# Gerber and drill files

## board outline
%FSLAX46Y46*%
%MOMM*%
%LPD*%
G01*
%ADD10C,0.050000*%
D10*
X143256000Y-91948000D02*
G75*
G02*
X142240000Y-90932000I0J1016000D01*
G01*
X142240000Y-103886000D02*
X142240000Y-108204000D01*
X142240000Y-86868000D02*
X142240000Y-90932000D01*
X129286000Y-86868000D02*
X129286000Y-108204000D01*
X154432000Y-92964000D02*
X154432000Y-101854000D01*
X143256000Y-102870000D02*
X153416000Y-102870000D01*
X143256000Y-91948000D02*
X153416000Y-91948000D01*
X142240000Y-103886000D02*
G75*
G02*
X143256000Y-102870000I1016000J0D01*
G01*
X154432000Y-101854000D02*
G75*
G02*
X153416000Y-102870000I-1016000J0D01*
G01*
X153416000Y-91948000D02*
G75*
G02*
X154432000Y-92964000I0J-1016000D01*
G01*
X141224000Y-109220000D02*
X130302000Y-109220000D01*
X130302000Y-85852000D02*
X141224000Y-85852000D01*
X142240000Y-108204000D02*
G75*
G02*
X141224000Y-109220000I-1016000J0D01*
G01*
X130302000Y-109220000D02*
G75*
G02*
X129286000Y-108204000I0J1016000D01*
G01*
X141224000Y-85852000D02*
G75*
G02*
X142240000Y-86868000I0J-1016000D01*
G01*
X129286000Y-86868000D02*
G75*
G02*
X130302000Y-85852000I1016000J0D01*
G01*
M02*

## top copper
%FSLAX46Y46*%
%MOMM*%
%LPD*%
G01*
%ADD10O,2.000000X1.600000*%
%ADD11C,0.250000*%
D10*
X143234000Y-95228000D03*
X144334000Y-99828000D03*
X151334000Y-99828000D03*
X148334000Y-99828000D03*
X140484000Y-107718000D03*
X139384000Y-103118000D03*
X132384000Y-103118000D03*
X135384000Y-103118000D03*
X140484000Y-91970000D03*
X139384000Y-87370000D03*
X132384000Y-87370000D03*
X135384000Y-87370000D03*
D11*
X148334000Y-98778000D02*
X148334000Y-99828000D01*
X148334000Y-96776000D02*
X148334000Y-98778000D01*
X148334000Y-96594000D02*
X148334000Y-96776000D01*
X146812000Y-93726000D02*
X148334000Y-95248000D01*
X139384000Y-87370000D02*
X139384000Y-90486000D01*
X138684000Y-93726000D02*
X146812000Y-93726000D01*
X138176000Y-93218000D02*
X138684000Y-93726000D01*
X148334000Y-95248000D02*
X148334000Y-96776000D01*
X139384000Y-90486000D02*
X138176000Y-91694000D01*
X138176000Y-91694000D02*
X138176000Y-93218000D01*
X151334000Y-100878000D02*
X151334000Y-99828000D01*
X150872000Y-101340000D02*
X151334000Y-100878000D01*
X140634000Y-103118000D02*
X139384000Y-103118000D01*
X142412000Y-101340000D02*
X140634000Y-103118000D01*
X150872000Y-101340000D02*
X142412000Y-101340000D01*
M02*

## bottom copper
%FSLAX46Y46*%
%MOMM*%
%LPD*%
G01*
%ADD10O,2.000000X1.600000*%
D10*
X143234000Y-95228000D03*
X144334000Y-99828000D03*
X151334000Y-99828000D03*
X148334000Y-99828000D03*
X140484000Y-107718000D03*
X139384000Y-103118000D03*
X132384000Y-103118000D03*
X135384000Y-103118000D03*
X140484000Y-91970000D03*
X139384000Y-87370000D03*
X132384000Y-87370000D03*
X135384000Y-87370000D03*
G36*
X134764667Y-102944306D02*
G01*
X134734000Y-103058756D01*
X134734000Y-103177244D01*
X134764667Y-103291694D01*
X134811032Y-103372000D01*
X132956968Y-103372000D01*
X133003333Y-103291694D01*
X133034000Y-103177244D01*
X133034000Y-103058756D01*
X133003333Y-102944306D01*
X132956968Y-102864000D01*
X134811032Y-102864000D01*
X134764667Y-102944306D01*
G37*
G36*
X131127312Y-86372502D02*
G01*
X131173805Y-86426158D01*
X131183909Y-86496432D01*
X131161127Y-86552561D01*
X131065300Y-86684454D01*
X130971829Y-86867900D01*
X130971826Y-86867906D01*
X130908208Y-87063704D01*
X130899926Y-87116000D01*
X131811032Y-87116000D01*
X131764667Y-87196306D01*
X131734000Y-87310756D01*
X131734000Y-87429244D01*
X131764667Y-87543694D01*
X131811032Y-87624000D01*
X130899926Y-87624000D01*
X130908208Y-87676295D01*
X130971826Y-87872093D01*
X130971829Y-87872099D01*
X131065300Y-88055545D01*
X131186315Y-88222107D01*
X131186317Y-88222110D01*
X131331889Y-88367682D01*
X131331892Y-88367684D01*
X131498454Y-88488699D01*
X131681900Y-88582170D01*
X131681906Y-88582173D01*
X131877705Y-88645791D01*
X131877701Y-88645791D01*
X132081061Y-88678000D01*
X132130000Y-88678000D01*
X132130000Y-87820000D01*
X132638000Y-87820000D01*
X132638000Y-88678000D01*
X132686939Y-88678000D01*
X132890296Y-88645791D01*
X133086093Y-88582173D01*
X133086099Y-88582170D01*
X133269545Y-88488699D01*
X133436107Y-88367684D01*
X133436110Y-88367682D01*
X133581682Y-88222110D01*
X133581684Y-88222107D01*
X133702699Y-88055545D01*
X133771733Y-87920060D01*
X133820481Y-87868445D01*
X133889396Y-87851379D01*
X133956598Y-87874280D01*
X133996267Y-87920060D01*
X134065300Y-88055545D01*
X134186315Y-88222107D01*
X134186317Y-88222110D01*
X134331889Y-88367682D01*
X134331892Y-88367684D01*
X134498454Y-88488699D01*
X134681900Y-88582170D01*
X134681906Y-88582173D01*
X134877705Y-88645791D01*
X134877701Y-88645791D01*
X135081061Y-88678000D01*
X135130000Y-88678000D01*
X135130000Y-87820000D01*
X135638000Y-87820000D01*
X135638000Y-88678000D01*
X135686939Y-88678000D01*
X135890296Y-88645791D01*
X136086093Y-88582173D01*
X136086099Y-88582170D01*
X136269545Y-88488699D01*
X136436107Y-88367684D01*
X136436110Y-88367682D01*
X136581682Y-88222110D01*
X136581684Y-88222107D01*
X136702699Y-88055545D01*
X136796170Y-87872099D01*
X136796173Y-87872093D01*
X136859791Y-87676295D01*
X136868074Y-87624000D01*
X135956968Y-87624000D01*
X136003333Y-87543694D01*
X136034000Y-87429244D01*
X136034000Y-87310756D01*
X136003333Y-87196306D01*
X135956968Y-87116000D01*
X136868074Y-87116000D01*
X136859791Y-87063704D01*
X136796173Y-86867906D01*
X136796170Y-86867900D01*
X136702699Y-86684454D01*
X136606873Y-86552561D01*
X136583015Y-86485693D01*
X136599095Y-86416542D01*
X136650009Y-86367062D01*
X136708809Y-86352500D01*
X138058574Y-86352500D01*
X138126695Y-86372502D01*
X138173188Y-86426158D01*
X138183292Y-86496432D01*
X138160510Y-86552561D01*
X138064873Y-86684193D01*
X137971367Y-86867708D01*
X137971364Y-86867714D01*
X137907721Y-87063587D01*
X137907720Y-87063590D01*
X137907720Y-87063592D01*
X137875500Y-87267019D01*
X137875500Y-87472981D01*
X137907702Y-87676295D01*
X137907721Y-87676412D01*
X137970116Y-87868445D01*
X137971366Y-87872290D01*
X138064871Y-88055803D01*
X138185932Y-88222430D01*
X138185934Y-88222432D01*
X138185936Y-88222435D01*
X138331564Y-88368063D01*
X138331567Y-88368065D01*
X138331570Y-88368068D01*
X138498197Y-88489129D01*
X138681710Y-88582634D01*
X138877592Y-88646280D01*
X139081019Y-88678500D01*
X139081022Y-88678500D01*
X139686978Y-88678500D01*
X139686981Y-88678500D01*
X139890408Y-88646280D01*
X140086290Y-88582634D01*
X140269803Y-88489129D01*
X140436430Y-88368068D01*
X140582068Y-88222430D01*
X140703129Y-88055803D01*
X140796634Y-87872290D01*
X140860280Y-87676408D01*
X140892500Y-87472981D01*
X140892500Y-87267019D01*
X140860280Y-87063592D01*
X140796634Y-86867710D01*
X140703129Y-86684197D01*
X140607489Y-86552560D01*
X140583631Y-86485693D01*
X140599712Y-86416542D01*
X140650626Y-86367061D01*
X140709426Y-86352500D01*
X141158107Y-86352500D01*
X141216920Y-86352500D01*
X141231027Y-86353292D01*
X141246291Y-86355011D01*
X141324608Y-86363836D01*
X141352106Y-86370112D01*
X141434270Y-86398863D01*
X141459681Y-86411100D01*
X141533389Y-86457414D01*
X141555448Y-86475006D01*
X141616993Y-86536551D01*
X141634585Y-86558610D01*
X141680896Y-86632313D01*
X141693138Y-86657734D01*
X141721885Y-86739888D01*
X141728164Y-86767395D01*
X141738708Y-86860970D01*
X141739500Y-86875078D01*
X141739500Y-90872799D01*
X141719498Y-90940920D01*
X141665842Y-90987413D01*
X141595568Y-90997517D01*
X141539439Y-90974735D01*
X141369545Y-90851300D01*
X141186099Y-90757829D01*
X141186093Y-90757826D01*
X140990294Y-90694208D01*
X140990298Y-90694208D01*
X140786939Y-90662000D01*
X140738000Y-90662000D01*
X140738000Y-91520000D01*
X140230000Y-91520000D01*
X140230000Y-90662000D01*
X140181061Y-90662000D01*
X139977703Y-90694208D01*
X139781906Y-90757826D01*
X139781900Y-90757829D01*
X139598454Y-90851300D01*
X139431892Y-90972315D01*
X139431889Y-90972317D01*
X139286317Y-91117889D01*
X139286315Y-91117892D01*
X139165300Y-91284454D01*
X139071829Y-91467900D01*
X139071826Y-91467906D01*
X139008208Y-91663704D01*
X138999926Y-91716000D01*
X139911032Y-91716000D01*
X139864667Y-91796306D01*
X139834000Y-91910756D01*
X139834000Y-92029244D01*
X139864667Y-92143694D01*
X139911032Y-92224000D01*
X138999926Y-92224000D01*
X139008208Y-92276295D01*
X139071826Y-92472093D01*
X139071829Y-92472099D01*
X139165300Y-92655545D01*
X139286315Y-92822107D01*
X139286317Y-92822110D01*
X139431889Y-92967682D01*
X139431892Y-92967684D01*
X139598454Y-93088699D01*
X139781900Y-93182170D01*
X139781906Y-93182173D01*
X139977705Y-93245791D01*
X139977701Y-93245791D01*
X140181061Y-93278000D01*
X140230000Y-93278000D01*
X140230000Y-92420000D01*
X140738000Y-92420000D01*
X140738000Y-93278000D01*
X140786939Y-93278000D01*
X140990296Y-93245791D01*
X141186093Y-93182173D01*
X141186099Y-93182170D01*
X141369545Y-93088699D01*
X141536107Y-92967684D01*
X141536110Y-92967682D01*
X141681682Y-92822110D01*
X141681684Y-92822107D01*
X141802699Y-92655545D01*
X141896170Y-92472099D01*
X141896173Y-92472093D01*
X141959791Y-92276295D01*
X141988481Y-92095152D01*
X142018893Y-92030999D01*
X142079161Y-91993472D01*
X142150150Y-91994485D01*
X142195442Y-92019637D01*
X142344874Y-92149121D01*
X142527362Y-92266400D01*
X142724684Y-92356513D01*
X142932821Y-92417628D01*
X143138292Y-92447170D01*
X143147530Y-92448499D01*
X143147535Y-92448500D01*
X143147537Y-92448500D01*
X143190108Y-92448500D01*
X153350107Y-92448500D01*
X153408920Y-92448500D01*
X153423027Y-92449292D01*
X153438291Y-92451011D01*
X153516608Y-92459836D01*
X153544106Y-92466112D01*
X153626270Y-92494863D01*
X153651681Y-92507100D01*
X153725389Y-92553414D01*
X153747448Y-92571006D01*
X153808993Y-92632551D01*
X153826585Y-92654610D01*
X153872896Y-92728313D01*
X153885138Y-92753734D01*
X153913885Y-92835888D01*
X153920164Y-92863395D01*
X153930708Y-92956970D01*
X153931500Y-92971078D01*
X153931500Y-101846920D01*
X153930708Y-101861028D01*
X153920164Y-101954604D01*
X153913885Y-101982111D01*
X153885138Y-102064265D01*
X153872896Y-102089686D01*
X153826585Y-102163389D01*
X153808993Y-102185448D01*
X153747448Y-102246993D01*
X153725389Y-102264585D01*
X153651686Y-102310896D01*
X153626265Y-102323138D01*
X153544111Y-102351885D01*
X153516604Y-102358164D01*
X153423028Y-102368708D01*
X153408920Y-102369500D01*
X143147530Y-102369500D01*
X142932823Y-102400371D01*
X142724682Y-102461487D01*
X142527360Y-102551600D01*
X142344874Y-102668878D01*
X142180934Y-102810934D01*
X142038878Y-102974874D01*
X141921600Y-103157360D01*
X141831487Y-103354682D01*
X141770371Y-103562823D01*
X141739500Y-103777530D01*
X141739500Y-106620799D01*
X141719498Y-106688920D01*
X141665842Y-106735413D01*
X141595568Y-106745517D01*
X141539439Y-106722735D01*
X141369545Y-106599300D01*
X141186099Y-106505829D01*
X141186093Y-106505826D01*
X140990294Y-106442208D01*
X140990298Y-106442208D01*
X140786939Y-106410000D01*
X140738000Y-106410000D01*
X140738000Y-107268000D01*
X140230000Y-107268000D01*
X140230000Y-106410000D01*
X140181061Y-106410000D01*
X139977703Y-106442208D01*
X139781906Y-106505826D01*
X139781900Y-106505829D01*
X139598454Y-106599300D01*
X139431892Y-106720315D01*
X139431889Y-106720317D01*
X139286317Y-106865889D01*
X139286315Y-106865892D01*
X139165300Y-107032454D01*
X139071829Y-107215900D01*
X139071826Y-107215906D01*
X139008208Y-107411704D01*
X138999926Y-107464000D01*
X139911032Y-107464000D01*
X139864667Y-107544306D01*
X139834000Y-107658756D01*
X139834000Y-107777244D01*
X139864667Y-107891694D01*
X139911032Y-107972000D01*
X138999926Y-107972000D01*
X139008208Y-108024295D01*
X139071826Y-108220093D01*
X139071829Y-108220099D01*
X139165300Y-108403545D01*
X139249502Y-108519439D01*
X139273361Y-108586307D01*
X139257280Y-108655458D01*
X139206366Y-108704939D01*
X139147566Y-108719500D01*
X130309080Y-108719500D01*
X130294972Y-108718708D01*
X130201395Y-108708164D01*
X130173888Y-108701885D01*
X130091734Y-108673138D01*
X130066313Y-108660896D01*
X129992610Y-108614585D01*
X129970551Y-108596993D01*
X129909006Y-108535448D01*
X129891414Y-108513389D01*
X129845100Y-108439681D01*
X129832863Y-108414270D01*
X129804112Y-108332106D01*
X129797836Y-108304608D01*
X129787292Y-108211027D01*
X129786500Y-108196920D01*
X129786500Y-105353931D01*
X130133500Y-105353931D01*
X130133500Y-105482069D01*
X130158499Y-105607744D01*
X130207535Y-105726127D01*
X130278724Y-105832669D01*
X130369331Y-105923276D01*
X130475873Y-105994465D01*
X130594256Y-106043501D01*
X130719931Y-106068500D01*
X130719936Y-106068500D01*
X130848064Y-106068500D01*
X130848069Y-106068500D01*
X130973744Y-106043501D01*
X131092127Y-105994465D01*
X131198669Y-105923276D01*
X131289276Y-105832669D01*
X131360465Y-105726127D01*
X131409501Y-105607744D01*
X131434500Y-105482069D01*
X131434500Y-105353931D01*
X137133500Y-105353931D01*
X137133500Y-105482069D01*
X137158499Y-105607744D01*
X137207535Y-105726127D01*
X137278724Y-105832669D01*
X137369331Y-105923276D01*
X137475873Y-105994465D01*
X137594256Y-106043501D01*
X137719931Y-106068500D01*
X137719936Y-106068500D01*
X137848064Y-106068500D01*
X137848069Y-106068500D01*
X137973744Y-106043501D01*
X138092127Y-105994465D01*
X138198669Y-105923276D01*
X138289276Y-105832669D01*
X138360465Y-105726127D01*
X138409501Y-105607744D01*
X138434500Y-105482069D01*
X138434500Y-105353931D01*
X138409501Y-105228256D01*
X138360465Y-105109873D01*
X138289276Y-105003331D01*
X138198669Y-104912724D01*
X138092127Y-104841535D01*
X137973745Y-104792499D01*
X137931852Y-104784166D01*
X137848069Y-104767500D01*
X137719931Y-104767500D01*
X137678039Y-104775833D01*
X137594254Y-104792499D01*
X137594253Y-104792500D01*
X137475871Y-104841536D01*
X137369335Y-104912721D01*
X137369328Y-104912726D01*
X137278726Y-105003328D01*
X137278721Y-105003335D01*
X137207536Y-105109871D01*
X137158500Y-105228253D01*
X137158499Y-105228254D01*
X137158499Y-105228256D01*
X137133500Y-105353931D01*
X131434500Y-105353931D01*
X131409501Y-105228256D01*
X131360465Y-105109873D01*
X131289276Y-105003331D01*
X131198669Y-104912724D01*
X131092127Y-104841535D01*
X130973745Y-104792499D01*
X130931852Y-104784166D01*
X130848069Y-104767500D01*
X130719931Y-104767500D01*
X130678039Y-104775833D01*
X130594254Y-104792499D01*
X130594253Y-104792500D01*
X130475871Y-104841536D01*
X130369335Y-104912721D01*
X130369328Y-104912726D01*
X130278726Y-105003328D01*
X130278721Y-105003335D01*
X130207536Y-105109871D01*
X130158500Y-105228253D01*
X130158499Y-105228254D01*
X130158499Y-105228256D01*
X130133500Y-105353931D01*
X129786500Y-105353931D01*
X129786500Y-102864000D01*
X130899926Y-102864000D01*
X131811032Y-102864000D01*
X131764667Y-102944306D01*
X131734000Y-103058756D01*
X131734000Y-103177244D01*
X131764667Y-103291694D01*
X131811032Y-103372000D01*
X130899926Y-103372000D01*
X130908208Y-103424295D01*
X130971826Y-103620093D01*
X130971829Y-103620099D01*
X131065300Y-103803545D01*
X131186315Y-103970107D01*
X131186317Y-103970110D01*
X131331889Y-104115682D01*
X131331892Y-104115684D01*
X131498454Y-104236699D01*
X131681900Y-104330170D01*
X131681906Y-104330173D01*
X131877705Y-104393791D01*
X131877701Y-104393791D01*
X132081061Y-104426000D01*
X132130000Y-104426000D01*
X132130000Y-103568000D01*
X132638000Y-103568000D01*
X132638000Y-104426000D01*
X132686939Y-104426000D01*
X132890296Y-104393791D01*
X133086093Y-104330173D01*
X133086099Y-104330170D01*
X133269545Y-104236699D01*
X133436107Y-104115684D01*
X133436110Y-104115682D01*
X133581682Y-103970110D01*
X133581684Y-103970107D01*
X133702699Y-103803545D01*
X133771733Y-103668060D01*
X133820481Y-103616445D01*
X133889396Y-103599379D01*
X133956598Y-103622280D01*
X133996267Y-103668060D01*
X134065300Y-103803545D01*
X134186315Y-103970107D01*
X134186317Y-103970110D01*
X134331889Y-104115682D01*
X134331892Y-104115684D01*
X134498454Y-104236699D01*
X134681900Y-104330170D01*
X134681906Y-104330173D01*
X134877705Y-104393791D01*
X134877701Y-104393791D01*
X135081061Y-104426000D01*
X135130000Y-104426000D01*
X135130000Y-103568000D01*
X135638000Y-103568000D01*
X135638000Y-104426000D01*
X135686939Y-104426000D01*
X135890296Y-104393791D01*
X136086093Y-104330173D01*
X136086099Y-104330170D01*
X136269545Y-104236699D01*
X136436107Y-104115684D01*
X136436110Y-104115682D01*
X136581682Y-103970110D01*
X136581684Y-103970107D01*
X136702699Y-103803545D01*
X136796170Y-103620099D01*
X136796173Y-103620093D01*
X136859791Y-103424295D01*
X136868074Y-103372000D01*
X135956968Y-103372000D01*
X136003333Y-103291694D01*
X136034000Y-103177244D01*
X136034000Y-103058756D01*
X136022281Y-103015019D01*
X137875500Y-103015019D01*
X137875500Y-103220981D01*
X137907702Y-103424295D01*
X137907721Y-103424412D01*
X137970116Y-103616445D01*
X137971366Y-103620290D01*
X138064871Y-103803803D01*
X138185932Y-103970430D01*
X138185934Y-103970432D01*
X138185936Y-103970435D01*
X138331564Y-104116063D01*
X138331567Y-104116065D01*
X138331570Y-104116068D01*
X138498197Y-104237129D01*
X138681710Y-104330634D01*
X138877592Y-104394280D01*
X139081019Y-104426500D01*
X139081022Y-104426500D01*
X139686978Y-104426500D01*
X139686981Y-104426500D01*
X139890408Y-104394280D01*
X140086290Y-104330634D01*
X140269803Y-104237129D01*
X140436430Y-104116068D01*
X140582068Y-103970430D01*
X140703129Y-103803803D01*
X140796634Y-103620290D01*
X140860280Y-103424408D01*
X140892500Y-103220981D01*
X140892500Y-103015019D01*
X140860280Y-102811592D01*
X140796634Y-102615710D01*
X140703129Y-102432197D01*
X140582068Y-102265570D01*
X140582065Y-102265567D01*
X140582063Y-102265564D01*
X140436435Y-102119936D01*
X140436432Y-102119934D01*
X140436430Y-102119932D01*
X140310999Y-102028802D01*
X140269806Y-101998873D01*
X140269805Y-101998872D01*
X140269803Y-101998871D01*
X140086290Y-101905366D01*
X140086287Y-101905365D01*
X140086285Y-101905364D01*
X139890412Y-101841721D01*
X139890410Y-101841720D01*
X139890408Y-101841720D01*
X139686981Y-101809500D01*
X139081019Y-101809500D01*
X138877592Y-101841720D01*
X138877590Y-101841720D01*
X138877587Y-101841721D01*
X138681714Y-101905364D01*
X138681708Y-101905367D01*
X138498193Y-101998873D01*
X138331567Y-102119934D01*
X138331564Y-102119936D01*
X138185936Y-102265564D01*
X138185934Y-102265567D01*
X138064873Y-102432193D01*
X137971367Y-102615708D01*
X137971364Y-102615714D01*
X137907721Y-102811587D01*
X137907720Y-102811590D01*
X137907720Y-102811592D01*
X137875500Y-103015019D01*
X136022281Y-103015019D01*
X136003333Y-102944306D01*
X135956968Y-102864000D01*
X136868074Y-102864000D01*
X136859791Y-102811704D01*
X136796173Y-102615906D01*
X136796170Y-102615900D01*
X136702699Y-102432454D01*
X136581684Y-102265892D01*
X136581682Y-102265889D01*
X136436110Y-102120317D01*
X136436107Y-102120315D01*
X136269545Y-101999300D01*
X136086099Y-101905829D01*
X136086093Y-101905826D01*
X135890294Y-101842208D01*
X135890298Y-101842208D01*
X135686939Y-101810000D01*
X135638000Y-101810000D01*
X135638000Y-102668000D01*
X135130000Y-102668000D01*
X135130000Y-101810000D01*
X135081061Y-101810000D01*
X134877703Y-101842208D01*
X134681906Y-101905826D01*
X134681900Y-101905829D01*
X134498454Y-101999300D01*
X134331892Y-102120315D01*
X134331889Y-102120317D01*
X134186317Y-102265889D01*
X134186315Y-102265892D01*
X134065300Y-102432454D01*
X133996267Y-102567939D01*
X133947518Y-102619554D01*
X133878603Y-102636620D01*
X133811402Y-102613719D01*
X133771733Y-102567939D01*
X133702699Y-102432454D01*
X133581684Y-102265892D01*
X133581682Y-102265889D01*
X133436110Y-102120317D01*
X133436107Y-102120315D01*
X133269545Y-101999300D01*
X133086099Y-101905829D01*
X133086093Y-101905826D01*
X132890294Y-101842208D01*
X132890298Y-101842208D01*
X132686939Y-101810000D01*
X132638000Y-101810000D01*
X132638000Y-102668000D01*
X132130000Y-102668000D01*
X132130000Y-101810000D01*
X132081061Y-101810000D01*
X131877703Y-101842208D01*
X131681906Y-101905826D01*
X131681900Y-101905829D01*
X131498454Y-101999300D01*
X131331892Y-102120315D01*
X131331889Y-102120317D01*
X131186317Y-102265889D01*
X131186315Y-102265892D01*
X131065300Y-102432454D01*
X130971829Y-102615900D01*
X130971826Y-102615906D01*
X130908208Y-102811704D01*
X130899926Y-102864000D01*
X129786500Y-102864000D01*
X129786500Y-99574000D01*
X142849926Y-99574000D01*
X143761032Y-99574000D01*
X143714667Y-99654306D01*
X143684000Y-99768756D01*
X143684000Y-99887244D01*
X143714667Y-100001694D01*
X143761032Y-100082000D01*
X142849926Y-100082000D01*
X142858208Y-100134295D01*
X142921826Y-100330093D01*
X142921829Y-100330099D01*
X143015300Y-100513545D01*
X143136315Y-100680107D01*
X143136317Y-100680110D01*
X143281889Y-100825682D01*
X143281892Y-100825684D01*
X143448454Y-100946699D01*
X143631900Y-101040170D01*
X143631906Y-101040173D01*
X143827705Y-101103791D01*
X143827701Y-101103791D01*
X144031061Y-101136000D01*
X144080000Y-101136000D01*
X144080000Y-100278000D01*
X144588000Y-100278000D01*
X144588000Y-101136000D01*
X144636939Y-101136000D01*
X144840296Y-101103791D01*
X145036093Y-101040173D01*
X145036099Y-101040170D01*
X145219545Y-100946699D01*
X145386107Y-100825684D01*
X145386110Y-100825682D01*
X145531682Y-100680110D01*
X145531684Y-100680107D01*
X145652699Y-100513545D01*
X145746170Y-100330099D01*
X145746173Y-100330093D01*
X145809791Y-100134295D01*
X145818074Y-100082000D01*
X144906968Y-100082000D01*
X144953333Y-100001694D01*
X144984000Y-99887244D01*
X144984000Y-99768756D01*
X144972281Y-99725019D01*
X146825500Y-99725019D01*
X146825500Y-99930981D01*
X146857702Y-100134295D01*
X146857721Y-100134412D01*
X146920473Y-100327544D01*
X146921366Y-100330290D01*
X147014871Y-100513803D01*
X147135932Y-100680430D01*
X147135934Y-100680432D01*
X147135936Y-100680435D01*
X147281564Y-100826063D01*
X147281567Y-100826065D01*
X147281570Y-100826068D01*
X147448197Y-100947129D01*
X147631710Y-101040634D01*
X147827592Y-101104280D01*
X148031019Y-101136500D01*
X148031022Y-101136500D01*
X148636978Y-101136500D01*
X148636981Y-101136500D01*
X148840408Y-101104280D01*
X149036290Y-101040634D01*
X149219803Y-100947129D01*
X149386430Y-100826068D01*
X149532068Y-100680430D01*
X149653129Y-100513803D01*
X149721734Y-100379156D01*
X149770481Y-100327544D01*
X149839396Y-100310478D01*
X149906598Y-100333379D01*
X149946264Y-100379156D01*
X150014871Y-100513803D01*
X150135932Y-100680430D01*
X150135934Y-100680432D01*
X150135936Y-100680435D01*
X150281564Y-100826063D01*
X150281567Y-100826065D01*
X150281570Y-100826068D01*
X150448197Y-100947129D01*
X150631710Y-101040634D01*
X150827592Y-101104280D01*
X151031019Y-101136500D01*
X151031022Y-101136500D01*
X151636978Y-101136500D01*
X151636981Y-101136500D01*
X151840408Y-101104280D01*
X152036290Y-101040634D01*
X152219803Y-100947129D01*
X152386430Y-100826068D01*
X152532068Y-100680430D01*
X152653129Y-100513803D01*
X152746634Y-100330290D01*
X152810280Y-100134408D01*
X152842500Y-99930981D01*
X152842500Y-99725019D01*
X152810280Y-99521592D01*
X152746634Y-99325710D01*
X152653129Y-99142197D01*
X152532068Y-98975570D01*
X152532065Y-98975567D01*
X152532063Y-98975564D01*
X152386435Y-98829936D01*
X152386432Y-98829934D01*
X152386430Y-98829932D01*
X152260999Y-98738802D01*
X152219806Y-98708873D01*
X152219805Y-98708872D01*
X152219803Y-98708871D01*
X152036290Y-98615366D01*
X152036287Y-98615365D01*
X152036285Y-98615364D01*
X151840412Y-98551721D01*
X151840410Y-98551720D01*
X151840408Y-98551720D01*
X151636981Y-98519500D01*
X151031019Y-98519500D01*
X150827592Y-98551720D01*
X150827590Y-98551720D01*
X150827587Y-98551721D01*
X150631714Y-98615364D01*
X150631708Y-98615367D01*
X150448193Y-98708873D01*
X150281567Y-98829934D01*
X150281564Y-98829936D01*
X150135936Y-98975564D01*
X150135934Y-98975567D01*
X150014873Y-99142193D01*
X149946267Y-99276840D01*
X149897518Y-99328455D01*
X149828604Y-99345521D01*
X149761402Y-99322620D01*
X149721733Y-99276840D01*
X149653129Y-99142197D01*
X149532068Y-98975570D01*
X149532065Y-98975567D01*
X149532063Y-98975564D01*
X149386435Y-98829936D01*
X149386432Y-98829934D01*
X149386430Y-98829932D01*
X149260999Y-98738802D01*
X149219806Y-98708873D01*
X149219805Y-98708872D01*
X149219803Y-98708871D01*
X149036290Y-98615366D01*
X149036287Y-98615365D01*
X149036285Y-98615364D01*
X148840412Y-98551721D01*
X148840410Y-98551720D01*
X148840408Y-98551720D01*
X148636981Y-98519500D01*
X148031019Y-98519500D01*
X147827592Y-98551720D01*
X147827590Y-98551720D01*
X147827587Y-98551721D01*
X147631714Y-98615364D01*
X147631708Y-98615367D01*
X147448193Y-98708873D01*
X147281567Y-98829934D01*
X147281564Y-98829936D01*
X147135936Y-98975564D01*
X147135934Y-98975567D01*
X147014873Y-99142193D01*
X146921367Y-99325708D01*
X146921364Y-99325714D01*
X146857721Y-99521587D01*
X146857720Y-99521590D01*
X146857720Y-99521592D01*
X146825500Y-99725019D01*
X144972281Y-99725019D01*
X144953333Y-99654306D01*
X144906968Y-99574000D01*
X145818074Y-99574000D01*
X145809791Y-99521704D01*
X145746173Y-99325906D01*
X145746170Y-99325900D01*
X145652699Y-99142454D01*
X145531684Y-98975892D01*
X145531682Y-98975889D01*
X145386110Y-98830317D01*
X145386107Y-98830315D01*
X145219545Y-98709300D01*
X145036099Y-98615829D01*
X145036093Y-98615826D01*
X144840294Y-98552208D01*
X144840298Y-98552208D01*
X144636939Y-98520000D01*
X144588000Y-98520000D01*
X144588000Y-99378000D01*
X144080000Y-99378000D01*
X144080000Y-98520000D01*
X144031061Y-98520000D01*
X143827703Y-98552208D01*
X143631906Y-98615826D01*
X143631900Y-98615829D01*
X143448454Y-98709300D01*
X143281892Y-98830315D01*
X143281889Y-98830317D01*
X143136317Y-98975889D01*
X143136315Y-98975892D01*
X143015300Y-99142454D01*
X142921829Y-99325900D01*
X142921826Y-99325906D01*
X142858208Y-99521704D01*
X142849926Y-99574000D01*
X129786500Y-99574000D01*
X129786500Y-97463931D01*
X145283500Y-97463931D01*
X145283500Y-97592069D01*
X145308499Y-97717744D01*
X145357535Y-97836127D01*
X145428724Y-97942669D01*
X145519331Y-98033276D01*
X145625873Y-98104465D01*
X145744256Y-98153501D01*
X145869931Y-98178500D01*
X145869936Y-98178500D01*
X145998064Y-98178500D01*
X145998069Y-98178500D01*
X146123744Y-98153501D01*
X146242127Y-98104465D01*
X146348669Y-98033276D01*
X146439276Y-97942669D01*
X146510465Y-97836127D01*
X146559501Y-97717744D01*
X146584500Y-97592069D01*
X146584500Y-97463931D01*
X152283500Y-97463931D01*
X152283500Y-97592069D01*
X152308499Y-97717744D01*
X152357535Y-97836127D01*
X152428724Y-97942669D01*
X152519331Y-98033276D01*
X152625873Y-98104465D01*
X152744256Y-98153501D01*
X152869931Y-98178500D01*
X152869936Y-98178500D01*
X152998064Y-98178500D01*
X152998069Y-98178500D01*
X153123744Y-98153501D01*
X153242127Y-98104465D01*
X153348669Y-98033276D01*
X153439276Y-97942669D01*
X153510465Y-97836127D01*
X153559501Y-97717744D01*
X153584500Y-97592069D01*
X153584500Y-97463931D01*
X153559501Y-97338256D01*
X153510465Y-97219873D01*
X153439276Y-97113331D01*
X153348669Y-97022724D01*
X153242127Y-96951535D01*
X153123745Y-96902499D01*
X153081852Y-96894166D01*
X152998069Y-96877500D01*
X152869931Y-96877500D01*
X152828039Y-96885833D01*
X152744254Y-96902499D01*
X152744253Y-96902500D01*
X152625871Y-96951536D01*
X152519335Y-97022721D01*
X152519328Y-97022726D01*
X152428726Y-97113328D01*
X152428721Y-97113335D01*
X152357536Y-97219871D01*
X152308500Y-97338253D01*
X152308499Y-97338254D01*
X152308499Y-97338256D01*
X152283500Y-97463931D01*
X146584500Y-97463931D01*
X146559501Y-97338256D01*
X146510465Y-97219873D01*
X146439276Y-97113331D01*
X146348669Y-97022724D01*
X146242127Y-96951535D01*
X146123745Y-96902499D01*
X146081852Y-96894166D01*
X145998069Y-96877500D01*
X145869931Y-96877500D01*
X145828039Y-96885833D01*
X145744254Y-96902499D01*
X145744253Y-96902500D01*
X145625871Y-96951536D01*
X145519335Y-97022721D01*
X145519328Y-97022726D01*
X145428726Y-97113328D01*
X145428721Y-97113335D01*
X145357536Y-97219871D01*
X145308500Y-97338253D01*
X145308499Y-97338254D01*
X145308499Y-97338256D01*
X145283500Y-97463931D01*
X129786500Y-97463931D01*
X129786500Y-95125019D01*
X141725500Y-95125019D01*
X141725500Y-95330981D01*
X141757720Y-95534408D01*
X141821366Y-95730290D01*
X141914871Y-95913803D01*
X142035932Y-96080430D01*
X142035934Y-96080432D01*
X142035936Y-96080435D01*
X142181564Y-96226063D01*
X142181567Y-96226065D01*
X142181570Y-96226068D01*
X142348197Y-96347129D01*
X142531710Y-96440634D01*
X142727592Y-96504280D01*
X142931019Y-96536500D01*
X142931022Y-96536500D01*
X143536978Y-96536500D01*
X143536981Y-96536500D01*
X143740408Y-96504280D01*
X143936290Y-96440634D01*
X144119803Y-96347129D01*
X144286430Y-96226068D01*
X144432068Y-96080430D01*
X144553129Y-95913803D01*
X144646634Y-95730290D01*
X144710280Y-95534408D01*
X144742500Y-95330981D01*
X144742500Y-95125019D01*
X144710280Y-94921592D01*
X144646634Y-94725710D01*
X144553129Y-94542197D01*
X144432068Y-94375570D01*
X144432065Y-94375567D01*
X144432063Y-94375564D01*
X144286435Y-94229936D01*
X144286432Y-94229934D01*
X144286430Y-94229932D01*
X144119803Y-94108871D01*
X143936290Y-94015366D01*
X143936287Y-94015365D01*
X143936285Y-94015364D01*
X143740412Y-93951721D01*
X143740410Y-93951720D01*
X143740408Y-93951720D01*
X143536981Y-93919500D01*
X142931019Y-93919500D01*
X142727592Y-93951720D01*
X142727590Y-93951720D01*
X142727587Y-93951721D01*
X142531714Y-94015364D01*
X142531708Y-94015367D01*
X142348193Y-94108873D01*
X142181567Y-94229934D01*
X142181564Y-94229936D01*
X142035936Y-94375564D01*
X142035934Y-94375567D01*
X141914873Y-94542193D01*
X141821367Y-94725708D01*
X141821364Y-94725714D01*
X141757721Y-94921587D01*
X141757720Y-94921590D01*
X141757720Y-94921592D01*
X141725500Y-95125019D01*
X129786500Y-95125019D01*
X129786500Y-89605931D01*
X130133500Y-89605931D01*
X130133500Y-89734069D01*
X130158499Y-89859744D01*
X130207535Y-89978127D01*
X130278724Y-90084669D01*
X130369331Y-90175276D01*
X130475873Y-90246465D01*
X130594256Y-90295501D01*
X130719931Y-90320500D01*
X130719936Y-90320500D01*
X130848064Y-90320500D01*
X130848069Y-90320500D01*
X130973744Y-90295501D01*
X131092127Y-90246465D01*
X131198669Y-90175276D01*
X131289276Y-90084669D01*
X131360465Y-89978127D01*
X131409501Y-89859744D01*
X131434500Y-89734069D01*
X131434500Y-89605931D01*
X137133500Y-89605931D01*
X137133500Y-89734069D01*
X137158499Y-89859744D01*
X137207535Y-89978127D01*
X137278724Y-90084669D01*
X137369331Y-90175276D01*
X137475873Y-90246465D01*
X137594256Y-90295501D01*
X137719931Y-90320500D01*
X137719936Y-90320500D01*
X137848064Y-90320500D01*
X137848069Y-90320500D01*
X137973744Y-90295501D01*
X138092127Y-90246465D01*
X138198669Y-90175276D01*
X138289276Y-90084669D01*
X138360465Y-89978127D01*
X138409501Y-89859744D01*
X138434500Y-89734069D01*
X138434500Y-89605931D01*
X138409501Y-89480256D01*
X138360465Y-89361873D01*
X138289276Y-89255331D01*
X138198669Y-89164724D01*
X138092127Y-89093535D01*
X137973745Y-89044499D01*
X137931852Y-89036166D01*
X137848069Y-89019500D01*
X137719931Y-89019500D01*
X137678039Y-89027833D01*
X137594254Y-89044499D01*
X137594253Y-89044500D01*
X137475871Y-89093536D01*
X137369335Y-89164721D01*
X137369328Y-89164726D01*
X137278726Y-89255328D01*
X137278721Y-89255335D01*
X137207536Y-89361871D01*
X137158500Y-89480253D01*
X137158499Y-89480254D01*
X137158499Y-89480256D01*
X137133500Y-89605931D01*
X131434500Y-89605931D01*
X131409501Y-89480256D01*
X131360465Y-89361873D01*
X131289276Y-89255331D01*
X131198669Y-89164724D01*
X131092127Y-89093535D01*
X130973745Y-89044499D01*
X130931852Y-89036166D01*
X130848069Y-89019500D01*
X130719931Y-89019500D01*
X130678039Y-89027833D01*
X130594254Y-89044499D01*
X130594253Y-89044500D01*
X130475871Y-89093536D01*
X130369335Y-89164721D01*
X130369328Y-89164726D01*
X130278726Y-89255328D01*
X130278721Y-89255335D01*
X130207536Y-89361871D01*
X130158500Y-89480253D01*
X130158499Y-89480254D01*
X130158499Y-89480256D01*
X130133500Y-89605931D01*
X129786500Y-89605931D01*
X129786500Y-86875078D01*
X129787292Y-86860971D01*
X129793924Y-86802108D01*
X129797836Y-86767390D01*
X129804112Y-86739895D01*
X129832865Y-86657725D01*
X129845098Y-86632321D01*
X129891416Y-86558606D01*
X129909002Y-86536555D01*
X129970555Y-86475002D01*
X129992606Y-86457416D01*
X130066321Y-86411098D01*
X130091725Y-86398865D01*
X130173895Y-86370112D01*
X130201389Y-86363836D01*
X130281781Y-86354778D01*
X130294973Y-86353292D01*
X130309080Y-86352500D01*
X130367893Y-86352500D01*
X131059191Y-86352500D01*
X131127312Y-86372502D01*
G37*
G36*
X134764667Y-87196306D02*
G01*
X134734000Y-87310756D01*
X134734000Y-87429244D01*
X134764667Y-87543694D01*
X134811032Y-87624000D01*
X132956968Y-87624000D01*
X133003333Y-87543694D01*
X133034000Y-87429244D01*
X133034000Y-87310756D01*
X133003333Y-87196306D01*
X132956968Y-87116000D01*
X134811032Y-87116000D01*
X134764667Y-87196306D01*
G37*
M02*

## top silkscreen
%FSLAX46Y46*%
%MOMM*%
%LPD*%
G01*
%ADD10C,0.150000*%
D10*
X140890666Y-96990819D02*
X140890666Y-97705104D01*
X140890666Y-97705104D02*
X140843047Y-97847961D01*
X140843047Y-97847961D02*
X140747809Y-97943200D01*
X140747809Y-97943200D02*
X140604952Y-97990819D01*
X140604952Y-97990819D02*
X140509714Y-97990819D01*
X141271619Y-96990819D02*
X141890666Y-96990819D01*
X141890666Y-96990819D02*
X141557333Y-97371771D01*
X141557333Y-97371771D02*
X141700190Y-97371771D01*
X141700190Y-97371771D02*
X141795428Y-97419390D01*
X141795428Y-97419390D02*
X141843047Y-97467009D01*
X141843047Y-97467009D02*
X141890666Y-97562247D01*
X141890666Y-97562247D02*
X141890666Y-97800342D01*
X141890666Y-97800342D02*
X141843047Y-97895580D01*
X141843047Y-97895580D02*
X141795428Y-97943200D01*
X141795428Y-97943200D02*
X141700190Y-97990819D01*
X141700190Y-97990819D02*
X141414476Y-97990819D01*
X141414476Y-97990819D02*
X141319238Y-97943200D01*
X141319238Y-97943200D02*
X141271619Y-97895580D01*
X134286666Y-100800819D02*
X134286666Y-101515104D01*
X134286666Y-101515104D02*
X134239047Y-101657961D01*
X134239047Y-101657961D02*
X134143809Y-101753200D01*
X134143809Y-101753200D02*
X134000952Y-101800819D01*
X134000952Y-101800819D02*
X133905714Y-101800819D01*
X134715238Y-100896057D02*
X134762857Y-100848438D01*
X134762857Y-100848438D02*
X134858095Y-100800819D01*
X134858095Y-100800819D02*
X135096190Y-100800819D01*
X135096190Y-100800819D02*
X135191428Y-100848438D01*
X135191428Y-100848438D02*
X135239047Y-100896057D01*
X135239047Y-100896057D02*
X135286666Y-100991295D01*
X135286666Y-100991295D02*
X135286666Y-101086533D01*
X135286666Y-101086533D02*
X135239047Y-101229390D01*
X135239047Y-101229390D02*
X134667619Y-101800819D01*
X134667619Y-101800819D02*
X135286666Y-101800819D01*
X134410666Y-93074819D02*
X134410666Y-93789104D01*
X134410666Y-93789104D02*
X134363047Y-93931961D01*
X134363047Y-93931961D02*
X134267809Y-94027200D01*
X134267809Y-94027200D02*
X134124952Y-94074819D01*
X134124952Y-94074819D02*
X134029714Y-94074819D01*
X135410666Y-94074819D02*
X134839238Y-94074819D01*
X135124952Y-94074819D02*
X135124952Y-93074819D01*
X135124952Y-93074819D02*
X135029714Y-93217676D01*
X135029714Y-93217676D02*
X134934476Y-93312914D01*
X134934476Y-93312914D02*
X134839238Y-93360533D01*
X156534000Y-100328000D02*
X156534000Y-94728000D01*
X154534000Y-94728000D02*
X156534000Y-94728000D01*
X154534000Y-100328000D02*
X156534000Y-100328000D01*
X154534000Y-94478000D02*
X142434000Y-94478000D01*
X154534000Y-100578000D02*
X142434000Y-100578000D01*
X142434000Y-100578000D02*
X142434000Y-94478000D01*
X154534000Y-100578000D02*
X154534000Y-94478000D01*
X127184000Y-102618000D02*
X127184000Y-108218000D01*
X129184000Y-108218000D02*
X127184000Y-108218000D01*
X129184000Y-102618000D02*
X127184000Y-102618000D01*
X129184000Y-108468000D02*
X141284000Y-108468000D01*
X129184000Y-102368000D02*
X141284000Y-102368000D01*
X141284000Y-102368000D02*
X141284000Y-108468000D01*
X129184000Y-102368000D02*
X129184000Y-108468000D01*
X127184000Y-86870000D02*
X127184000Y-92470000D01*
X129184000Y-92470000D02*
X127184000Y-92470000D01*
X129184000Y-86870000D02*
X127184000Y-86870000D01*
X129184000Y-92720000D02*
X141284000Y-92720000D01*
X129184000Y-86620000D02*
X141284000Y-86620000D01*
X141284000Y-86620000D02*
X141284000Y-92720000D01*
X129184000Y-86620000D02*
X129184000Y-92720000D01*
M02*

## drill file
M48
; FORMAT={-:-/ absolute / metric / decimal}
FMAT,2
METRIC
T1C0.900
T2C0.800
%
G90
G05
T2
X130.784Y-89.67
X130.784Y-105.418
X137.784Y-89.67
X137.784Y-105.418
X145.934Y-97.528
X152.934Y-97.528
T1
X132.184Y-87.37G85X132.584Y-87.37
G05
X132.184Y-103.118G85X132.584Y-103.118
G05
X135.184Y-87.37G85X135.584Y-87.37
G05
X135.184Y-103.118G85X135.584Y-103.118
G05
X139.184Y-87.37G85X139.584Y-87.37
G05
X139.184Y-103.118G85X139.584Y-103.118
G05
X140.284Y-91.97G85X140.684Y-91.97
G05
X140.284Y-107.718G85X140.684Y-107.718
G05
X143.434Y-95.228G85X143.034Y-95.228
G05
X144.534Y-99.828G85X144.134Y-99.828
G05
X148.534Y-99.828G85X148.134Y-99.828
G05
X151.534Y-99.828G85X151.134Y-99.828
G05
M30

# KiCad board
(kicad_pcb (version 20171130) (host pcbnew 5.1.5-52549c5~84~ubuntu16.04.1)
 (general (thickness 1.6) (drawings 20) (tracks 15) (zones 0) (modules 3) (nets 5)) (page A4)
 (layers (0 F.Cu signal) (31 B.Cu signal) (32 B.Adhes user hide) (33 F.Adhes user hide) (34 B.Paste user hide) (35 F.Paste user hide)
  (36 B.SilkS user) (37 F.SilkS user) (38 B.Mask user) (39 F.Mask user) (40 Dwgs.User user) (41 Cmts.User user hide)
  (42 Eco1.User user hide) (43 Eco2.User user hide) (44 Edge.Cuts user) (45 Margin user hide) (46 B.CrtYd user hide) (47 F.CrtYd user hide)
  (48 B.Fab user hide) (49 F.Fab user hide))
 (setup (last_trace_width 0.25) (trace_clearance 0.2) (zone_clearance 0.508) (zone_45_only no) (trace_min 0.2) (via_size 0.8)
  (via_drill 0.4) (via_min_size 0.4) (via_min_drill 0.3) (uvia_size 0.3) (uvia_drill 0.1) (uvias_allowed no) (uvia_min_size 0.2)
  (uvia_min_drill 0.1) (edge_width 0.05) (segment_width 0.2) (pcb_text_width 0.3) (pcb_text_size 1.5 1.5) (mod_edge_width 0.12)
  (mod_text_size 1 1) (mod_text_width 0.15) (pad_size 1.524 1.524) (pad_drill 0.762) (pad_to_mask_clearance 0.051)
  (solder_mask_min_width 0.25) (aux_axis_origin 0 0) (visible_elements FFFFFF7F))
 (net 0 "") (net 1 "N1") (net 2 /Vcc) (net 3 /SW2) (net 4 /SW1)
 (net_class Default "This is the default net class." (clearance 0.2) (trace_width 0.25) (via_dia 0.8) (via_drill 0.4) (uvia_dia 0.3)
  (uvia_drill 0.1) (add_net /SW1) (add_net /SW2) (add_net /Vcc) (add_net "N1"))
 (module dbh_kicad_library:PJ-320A (layer F.Cu) (at 151.384 99.568 180)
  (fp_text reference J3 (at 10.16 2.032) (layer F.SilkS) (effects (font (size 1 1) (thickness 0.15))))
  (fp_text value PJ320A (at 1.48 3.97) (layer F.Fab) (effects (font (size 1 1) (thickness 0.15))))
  (fp_line (start -5.15 -0.76) (end -5.15 4.84) (layer F.SilkS) (width 0.15))
  (fp_line (start -3.15 4.84) (end -5.15 4.84) (layer F.SilkS) (width 0.15))
  (fp_line (start -3.15 -0.76) (end -5.15 -0.76) (layer F.SilkS) (width 0.15))
  (fp_line (start -3.15 5.09) (end 8.95 5.09) (layer F.SilkS) (width 0.15))
  (fp_line (start -3.15 -1.01) (end 8.95 -1.01) (layer F.SilkS) (width 0.15))
  (fp_line (start 8.95 -1.01) (end 8.95 5.09) (layer F.SilkS) (width 0.15))
  (fp_line (start -3.15 -1.01) (end -3.15 5.09) (layer F.SilkS) (width 0.15))
  (pad 5 thru_hole oval (at 8.15 4.34 270) (size 1.6 2) (drill oval 0.9 1.3) (layers *.Cu *.Mask) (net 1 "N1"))
  (pad 4 thru_hole oval (at 7.05 -0.26 270) (size 1.6 2) (drill oval 0.9 1.3) (layers *.Cu *.Mask) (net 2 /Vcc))
  (pad 2 thru_hole oval (at 0.05 -0.26 270) (size 1.6 2) (drill oval 0.9 1.3) (layers *.Cu *.Mask) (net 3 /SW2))
  (pad "" np_thru_hole circle (at 5.45 2.04 270) (size 0.8 0.8) (drill 0.8) (layers *.Cu *.Mask))
  (pad "" np_thru_hole circle (at -1.55 2.04 270) (size 0.8 0.8) (drill 0.8) (layers *.Cu *.Mask))
  (pad 3 thru_hole oval (at 3.05 -0.26 270) (size 1.6 2) (drill oval 0.9 1.3) (layers *.Cu *.Mask) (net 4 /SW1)))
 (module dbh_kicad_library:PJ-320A (layer F.Cu) (at 132.334 103.378)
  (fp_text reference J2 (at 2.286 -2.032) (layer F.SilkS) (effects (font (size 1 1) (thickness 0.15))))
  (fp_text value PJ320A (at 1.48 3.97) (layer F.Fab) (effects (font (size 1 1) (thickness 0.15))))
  (fp_line (start -5.15 -0.76) (end -5.15 4.84) (layer F.SilkS) (width 0.15))
  (fp_line (start -3.15 4.84) (end -5.15 4.84) (layer F.SilkS) (width 0.15))
  (fp_line (start -3.15 -0.76) (end -5.15 -0.76) (layer F.SilkS) (width 0.15))
  (fp_line (start -3.15 5.09) (end 8.95 5.09) (layer F.SilkS) (width 0.15))
  (fp_line (start -3.15 -1.01) (end 8.95 -1.01) (layer F.SilkS) (width 0.15))
  (fp_line (start 8.95 -1.01) (end 8.95 5.09) (layer F.SilkS) (width 0.15))
  (fp_line (start -3.15 -1.01) (end -3.15 5.09) (layer F.SilkS) (width 0.15))
  (pad 5 thru_hole oval (at 8.15 4.34 90) (size 1.6 2) (drill oval 0.9 1.3) (layers *.Cu *.Mask) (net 2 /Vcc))
  (pad 4 thru_hole oval (at 7.05 -0.26 90) (size 1.6 2) (drill oval 0.9 1.3) (layers *.Cu *.Mask) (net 3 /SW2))
  (pad 2 thru_hole oval (at 0.05 -0.26 90) (size 1.6 2) (drill oval 0.9 1.3) (layers *.Cu *.Mask) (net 2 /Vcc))
  (pad "" np_thru_hole circle (at 5.45 2.04 90) (size 0.8 0.8) (drill 0.8) (layers *.Cu *.Mask))
  (pad "" np_thru_hole circle (at -1.55 2.04 90) (size 0.8 0.8) (drill 0.8) (layers *.Cu *.Mask))
  (pad 3 thru_hole oval (at 3.05 -0.26 90) (size 1.6 2) (drill oval 0.9 1.3) (layers *.Cu *.Mask) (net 2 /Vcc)))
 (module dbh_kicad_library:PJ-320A (layer F.Cu) (at 132.334 87.63)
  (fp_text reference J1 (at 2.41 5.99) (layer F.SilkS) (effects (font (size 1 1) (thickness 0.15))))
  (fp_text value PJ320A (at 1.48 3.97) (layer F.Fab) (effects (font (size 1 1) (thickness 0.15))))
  (fp_line (start -5.15 -0.76) (end -5.15 4.84) (layer F.SilkS) (width 0.15))
  (fp_line (start -3.15 4.84) (end -5.15 4.84) (layer F.SilkS) (width 0.15))
  (fp_line (start -3.15 -0.76) (end -5.15 -0.76) (layer F.SilkS) (width 0.15))
  (fp_line (start -3.15 5.09) (end 8.95 5.09) (layer F.SilkS) (width 0.15))
  (fp_line (start -3.15 -1.01) (end 8.95 -1.01) (layer F.SilkS) (width 0.15))
  (fp_line (start 8.95 -1.01) (end 8.95 5.09) (layer F.SilkS) (width 0.15))
  (fp_line (start -3.15 -1.01) (end -3.15 5.09) (layer F.SilkS) (width 0.15))
  (pad 5 thru_hole oval (at 8.15 4.34 90) (size 1.6 2) (drill oval 0.9 1.3) (layers *.Cu *.Mask) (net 2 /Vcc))
  (pad 4 thru_hole oval (at 7.05 -0.26 90) (size 1.6 2) (drill oval 0.9 1.3) (layers *.Cu *.Mask) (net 4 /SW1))
  (pad 2 thru_hole oval (at 0.05 -0.26 90) (size 1.6 2) (drill oval 0.9 1.3) (layers *.Cu *.Mask) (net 2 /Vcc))
  (pad "" np_thru_hole circle (at 5.45 2.04 90) (size 0.8 0.8) (drill 0.8) (layers *.Cu *.Mask))
  (pad "" np_thru_hole circle (at -1.55 2.04 90) (size 0.8 0.8) (drill 0.8) (layers *.Cu *.Mask))
  (pad 3 thru_hole oval (at 3.05 -0.26 90) (size 1.6 2) (drill oval 0.9 1.3) (layers *.Cu *.Mask) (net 2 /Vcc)))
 (gr_arc (start 143.256 90.932) (end 142.24 90.932) (angle -90) (layer Edge.Cuts) (width 0.05))
 (gr_line (start 142.24 103.886) (end 142.24 108.204) (layer Edge.Cuts) (width 0.05))
 (gr_line (start 142.24 86.868) (end 142.24 90.932) (layer Edge.Cuts) (width 0.05))
 (gr_line (start 129.286 86.868) (end 129.286 108.204) (layer Edge.Cuts) (width 0.05))
 (gr_line (start 154.432 92.964) (end 154.432 101.854) (layer Edge.Cuts) (width 0.05))
 (gr_line (start 143.256 102.87) (end 153.416 102.87) (layer Edge.Cuts) (width 0.05))
 (gr_line (start 143.256 91.948) (end 153.416 91.948) (layer Edge.Cuts) (width 0.05))
 (gr_arc (start 143.256 103.886) (end 143.256 102.87) (angle -90) (layer Edge.Cuts) (width 0.05))
 (gr_arc (start 153.416 101.854) (end 153.416 102.87) (angle -90) (layer Edge.Cuts) (width 0.05))
 (gr_arc (start 153.416 92.964) (end 154.432 92.964) (angle -90) (layer Edge.Cuts) (width 0.05))
 (gr_line (start 141.224 109.22) (end 130.302 109.22) (layer Edge.Cuts) (width 0.05))
 (gr_line (start 130.302 85.852) (end 141.224 85.852) (layer Edge.Cuts) (width 0.05))
 (gr_arc (start 141.224 108.204) (end 142.24 108.204) (angle 90) (layer Edge.Cuts) (width 0.05))
 (gr_arc (start 130.302 108.204) (end 130.302 109.22) (angle 90) (layer Edge.Cuts) (width 0.05))
 (gr_arc (start 141.224 86.868) (end 142.24 86.868) (angle -90) (layer Edge.Cuts) (width 0.05))
 (gr_arc (start 130.302 86.868) (end 130.302 85.852) (angle -90) (layer Edge.Cuts) (width 0.05))
 (segment (start 148.334 98.778) (end 148.334 99.828) (width 0.25) (layer F.Cu) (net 4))
 (segment (start 148.334 96.776) (end 148.334 98.778) (width 0.25) (layer F.Cu) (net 4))
 (segment (start 148.334 96.594) (end 148.334 96.776) (width 0.25) (layer F.Cu) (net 4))
 (segment (start 146.812 93.726) (end 148.334 95.248) (width 0.25) (layer F.Cu) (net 4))
 (segment (start 139.384 87.37) (end 139.384 90.486) (width 0.25) (layer F.Cu) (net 4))
 (segment (start 138.684 93.726) (end 146.812 93.726) (width 0.25) (layer F.Cu) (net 4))
 (segment (start 138.176 93.218) (end 138.684 93.726) (width 0.25) (layer F.Cu) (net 4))
 (segment (start 148.334 95.248) (end 148.334 96.776) (width 0.25) (layer F.Cu) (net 4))
 (segment (start 139.384 90.486) (end 138.176 91.694) (width 0.25) (layer F.Cu) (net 4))
 (segment (start 138.176 91.694) (end 138.176 93.218) (width 0.25) (layer F.Cu) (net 4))
 (segment (start 151.334 100.878) (end 151.334 99.828) (width 0.25) (layer F.Cu) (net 3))
 (segment (start 150.872 101.34) (end 151.334 100.878) (width 0.25) (layer F.Cu) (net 3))
 (segment (start 140.634 103.118) (end 139.384 103.118) (width 0.25) (layer F.Cu) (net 3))
 (segment (start 142.412 101.34) (end 140.634 103.118) (width 0.25) (layer F.Cu) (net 3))
 (segment (start 150.872 101.34) (end 142.412 101.34) (width 0.25) (layer F.Cu) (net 3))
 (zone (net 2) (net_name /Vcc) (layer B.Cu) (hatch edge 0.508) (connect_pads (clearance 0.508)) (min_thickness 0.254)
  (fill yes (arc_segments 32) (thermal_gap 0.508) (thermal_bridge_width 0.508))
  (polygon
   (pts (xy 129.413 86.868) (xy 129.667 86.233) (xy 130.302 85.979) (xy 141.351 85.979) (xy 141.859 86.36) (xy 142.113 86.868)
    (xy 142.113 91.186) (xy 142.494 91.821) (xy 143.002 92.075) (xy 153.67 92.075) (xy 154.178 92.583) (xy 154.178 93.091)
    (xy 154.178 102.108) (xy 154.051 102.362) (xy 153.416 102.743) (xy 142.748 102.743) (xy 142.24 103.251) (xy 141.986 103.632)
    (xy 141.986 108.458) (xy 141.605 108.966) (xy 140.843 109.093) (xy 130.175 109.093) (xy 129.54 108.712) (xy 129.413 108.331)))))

